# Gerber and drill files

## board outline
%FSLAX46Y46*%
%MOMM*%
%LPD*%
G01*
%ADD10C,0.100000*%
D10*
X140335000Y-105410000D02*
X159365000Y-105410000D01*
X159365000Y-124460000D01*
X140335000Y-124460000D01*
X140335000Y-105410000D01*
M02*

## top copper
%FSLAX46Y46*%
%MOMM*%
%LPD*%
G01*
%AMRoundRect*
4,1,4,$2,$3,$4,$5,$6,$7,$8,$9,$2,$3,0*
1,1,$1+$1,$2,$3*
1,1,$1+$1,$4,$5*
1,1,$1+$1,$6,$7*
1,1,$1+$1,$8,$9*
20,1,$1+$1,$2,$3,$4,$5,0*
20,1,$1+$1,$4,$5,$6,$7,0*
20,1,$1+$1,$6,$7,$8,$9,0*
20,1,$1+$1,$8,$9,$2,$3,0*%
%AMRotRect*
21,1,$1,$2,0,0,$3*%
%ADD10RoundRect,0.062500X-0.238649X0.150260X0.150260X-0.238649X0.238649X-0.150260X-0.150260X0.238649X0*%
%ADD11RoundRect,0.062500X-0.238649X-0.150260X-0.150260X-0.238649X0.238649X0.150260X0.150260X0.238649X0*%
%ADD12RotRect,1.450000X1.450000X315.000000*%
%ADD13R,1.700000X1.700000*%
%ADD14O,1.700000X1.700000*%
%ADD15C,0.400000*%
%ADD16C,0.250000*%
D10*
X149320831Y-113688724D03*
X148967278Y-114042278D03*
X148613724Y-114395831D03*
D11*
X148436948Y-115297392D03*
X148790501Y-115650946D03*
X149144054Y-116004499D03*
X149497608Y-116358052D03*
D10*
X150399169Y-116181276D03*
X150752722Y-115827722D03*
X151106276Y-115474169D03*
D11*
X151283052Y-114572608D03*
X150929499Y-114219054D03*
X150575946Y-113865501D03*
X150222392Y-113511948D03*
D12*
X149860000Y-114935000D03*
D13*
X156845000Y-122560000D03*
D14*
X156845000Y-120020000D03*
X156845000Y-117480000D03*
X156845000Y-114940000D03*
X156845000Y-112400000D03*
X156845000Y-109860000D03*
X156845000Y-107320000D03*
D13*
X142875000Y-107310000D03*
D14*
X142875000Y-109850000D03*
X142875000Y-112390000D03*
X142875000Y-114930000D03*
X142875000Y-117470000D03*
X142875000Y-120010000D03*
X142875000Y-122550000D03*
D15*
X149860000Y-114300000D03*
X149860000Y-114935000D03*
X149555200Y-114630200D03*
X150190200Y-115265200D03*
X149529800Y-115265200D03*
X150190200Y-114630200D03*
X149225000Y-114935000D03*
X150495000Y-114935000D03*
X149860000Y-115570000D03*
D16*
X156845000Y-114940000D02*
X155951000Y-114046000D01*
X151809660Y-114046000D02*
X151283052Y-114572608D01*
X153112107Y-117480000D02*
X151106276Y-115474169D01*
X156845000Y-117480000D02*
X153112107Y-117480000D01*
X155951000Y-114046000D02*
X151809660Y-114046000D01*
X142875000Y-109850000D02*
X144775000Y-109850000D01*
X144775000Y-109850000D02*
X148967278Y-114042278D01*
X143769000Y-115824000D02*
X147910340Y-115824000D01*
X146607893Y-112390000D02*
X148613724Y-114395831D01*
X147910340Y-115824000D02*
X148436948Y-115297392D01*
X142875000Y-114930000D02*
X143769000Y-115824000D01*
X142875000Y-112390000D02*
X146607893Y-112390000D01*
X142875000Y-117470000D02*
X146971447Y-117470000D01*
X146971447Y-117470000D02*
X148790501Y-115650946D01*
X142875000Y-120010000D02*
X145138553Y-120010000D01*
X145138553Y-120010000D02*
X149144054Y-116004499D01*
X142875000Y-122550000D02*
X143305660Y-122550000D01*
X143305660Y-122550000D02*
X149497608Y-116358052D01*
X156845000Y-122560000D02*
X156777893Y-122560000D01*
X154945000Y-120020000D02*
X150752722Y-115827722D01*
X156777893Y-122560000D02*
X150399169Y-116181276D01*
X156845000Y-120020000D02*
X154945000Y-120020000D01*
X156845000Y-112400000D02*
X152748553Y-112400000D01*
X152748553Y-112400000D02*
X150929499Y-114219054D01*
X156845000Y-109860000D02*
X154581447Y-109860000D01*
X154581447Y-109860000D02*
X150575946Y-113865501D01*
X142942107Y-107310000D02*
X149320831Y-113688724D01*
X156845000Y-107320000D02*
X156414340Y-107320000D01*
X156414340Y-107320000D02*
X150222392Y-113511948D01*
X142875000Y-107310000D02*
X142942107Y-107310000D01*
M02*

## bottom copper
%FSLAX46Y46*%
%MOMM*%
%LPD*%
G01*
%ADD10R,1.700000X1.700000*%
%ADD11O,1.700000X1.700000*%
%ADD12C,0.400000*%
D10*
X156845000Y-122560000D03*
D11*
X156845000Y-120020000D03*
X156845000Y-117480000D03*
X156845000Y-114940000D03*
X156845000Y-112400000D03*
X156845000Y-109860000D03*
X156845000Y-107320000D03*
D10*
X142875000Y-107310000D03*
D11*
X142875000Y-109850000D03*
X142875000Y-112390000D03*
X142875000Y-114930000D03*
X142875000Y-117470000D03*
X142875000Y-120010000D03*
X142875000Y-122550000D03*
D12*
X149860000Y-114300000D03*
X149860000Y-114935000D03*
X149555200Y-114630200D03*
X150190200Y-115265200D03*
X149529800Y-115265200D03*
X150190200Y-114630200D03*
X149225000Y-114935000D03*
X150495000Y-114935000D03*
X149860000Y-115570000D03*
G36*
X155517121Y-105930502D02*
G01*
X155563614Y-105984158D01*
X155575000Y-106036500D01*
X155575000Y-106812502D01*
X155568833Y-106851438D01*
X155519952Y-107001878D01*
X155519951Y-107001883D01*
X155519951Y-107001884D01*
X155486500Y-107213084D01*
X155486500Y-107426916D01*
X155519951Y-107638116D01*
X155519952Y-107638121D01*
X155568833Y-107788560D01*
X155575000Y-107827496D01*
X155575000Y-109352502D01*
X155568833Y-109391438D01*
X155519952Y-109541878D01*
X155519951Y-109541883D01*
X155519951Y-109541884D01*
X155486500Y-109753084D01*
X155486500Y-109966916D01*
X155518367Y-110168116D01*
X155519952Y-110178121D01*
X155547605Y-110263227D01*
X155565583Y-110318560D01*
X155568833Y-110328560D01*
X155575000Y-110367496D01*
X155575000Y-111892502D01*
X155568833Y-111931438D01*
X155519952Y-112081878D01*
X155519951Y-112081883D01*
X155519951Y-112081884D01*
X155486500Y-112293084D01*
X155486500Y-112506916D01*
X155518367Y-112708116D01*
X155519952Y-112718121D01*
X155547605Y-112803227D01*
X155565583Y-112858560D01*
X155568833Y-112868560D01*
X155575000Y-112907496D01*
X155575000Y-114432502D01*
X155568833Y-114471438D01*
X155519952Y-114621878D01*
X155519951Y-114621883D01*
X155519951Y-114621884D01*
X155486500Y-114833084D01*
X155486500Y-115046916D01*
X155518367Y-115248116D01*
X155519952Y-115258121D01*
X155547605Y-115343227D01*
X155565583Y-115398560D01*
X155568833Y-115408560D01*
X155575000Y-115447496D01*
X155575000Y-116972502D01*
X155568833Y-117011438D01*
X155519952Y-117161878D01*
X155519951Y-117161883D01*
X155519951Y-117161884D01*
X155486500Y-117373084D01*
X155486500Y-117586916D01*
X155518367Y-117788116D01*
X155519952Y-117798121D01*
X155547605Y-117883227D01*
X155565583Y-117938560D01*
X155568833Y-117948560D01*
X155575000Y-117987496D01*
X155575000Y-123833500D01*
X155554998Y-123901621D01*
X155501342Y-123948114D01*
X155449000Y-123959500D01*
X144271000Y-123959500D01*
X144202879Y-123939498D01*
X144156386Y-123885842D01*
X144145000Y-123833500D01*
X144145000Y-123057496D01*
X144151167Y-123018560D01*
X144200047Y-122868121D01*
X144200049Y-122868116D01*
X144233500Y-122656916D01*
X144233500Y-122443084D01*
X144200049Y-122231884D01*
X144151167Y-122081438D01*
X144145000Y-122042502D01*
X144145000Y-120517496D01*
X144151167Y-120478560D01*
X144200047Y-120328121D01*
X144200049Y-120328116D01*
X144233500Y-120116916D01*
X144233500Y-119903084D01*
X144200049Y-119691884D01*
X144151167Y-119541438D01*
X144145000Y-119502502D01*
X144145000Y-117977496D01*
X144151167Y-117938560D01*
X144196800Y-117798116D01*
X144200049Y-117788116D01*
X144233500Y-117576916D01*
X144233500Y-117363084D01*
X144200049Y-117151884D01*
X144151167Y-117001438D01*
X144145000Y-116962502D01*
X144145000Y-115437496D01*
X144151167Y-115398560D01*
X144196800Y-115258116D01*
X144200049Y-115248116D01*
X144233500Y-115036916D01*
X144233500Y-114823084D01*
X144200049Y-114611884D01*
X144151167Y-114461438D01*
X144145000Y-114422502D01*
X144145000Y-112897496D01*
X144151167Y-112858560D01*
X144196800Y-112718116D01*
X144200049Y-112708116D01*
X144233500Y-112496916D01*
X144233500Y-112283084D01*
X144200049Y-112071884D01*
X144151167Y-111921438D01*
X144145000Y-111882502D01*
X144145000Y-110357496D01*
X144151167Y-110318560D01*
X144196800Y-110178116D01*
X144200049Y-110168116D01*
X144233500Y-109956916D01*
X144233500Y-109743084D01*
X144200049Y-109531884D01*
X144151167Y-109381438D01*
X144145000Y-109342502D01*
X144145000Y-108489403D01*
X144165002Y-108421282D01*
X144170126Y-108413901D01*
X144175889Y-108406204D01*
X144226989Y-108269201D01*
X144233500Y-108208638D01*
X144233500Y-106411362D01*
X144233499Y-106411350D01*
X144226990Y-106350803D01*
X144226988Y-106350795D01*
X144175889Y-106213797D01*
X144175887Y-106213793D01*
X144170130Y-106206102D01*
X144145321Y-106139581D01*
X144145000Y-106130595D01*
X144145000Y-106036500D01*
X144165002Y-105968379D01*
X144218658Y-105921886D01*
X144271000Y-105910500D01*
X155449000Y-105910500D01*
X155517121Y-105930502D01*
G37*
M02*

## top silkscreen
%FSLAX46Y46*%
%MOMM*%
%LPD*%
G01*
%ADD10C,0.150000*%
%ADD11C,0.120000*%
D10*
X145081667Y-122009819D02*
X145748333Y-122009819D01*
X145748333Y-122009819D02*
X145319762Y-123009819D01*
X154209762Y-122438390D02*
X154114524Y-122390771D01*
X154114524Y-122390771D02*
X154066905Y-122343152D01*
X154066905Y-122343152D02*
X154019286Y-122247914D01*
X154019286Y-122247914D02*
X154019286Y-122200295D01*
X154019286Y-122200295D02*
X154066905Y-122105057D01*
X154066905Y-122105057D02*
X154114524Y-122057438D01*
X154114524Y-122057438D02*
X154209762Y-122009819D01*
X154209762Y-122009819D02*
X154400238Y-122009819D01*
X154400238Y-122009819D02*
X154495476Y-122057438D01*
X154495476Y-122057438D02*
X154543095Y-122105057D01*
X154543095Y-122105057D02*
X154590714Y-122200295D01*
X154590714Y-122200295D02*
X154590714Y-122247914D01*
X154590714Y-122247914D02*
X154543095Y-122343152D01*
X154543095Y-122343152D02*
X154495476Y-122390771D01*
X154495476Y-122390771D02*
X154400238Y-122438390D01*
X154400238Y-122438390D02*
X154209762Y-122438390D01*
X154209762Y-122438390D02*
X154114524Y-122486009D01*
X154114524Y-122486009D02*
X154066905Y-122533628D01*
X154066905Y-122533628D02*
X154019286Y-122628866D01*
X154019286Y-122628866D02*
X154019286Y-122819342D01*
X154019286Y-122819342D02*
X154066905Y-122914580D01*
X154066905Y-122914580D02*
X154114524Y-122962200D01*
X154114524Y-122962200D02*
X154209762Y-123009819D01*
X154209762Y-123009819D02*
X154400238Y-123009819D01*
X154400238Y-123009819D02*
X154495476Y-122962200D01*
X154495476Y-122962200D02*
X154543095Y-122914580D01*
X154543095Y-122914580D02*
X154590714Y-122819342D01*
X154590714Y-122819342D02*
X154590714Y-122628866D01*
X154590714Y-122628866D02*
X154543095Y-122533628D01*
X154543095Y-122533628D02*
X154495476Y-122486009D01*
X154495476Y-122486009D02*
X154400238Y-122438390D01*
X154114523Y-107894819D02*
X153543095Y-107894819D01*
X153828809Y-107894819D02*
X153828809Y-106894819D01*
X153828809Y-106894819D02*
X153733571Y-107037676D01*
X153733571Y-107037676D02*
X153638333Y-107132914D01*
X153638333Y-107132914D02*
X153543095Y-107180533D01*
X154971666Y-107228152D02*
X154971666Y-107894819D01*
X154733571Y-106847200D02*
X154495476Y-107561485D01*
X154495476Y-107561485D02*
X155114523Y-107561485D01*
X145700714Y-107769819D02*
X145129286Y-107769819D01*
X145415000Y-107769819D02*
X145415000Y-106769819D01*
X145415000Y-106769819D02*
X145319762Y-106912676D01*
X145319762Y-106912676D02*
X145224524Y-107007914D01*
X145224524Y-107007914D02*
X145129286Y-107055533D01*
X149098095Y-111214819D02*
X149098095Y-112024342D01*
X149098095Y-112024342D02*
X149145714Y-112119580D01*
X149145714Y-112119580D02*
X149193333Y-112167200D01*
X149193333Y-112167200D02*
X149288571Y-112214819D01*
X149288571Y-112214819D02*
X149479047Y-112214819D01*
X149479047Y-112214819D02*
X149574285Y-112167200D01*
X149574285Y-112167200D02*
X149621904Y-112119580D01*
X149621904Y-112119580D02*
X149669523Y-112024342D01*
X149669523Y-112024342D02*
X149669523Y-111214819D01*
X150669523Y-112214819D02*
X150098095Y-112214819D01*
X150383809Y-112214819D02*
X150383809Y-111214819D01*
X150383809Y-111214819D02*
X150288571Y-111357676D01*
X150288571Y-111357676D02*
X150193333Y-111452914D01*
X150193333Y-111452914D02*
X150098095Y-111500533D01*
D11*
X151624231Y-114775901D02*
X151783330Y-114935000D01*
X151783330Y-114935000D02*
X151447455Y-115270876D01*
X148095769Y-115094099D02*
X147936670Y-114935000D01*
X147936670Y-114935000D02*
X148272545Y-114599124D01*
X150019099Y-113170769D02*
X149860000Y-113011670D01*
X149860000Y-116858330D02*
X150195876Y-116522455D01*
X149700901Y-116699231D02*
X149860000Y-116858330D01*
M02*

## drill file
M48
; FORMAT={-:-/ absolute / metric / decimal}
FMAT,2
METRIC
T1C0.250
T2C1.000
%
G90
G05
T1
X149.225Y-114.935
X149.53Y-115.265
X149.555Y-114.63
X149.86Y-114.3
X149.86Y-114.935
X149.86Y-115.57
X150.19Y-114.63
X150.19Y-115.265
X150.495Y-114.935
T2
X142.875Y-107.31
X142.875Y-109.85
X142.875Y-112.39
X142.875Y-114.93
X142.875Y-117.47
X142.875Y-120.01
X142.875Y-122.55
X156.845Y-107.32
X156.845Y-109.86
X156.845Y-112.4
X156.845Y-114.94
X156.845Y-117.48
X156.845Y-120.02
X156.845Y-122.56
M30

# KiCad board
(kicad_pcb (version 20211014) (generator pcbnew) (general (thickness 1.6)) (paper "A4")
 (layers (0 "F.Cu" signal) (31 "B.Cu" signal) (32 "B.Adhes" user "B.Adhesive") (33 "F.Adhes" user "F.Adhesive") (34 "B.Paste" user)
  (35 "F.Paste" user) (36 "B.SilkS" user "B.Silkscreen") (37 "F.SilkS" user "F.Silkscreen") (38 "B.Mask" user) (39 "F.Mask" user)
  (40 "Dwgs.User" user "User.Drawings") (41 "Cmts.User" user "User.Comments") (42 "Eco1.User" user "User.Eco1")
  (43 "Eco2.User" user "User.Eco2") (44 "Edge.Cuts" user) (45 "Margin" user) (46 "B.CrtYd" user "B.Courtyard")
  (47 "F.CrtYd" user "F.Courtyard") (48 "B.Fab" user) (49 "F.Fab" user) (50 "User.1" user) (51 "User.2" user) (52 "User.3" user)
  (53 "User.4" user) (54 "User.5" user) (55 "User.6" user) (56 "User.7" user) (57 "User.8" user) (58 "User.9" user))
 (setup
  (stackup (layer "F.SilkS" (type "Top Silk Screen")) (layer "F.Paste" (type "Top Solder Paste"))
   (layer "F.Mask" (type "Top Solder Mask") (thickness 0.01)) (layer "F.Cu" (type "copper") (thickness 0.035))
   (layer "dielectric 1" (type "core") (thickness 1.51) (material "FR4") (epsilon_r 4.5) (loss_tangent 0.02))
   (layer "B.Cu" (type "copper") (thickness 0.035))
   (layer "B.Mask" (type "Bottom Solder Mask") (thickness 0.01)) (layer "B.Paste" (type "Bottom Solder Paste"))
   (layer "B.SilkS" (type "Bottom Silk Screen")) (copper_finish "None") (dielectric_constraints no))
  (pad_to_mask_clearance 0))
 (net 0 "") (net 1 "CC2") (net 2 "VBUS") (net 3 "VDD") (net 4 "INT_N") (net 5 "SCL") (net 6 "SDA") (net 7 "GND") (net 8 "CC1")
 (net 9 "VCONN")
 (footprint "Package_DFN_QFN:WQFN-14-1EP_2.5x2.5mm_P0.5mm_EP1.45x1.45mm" (layer "F.Cu") (at 149.86 114.935 -45)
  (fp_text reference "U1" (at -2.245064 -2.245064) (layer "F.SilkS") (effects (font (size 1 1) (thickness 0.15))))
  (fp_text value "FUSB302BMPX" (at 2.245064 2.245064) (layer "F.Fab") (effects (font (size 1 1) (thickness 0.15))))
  (fp_line (start 1.135 -1.36) (end 1.36 -1.36) (layer "F.SilkS") (width 0.12))
  (fp_line (start 1.36 -1.36) (end 1.36 -0.885) (layer "F.SilkS") (width 0.12))
  (fp_line (start -1.135 1.36) (end -1.36 1.36) (layer "F.SilkS") (width 0.12))
  (fp_line (start -1.36 1.36) (end -1.36 0.885) (layer "F.SilkS") (width 0.12))
  (fp_line (start -1.135 -1.36) (end -1.36 -1.36) (layer "F.SilkS") (width 0.12))
  (fp_line (start 1.36 1.36) (end 1.36 0.885) (layer "F.SilkS") (width 0.12))
  (fp_line (start 1.135 1.36) (end 1.36 1.36) (layer "F.SilkS") (width 0.12))
  (pad "" smd roundrect (at -0.36 0.36 315) (size 0.58 0.58) (layers "F.Paste") (roundrect_rratio 0.25))
  (pad "" smd roundrect (at 0.36 0.36 315) (size 0.58 0.58) (layers "F.Paste") (roundrect_rratio 0.25))
  (pad "" smd roundrect (at 0.36 -0.36 315) (size 0.58 0.58) (layers "F.Paste") (roundrect_rratio 0.25))
  (pad "" smd roundrect (at -0.36 -0.36 315) (size 0.58 0.58) (layers "F.Paste") (roundrect_rratio 0.25))
  (pad "1" smd roundrect (at -1.2625 -0.5 315) (size 0.675 0.25) (layers "F.Cu" "F.Paste" "F.Mask") (roundrect_rratio 0.25) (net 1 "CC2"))
  (pad "2" smd roundrect (at -1.2625 0 315) (size 0.675 0.25) (layers "F.Cu" "F.Paste" "F.Mask") (roundrect_rratio 0.25) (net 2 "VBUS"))
  (pad "3" smd roundrect (at -1.2625 0.5 315) (size 0.675 0.25) (layers "F.Cu" "F.Paste" "F.Mask") (roundrect_rratio 0.25) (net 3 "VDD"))
  (pad "4" smd roundrect (at -0.75 1.2625 315) (size 0.25 0.675) (layers "F.Cu" "F.Paste" "F.Mask") (roundrect_rratio 0.25) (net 3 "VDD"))
  (pad "5" smd roundrect (at -0.25 1.2625 315) (size 0.25 0.675) (layers "F.Cu" "F.Paste" "F.Mask") (roundrect_rratio 0.25) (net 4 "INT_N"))
  (pad "6" smd roundrect (at 0.25 1.2625 315) (size 0.25 0.675) (layers "F.Cu" "F.Paste" "F.Mask") (roundrect_rratio 0.25) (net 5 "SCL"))
  (pad "7" smd roundrect (at 0.75 1.2625 315) (size 0.25 0.675) (layers "F.Cu" "F.Paste" "F.Mask") (roundrect_rratio 0.25) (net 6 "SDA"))
  (pad "8" smd roundrect (at 1.2625 0.5 315) (size 0.675 0.25) (layers "F.Cu" "F.Paste" "F.Mask") (roundrect_rratio 0.25) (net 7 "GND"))
  (pad "9" smd roundrect (at 1.2625 0 315) (size 0.675 0.25) (layers "F.Cu" "F.Paste" "F.Mask") (roundrect_rratio 0.25) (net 7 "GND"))
  (pad "10" smd roundrect (at 1.2625 -0.5 315) (size 0.675 0.25) (layers "F.Cu" "F.Paste" "F.Mask") (roundrect_rratio 0.25) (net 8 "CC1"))
  (pad "11" smd roundrect (at 0.75 -1.2625 315) (size 0.25 0.675) (layers "F.Cu" "F.Paste" "F.Mask") (roundrect_rratio 0.25) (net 8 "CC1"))
  (pad "12" smd roundrect (at 0.25 -1.2625 315) (size 0.25 0.675) (layers "F.Cu" "F.Paste" "F.Mask") (roundrect_rratio 0.25) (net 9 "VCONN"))
  (pad "13" smd roundrect (at -0.25 -1.2625 315) (size 0.25 0.675) (layers "F.Cu" "F.Paste" "F.Mask") (roundrect_rratio 0.25)
   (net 9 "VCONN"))
  (pad "14" smd roundrect (at -0.75 -1.2625 315) (size 0.25 0.675) (layers "F.Cu" "F.Paste" "F.Mask") (roundrect_rratio 0.25) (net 1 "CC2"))
  (pad "15" smd rect (at 0 0 315) (size 1.45 1.45) (layers "F.Cu" "F.Mask") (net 7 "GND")))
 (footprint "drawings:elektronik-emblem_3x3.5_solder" (layer "B.Cu") (at 149.86 109.22 180)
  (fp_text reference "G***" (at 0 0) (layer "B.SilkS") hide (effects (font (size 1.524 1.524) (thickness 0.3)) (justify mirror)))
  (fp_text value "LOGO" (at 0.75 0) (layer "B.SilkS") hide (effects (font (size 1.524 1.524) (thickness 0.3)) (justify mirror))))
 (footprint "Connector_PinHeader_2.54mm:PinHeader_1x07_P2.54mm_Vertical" (layer "B.Cu") (at 156.845 122.56)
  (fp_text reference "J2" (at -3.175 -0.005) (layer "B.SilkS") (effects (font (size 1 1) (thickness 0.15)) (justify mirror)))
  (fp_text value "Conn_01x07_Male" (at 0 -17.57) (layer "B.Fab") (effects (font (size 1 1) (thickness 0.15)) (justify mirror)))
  (pad "1" thru_hole rect (at 0 0) (size 1.7 1.7) (drill 1) (layers *.Cu *.Mask) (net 7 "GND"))
  (pad "2" thru_hole oval (at 0 -2.54) (size 1.7 1.7) (drill 1) (layers *.Cu *.Mask) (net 7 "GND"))
  (pad "3" thru_hole oval (at 0 -5.08) (size 1.7 1.7) (drill 1) (layers *.Cu *.Mask) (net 8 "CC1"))
  (pad "4" thru_hole oval (at 0 -7.62) (size 1.7 1.7) (drill 1) (layers *.Cu *.Mask) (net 8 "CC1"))
  (pad "5" thru_hole oval (at 0 -10.16) (size 1.7 1.7) (drill 1) (layers *.Cu *.Mask) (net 9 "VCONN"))
  (pad "6" thru_hole oval (at 0 -12.7) (size 1.7 1.7) (drill 1) (layers *.Cu *.Mask) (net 9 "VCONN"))
  (pad "7" thru_hole oval (at 0 -15.24) (size 1.7 1.7) (drill 1) (layers *.Cu *.Mask) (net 1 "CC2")))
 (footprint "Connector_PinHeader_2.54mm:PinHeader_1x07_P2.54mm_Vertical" (layer "B.Cu") (at 142.875 107.31 180)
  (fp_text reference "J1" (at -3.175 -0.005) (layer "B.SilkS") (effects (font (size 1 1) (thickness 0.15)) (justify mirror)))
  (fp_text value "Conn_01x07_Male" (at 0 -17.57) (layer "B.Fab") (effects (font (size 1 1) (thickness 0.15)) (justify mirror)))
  (pad "1" thru_hole rect (at 0 0 180) (size 1.7 1.7) (drill 1) (layers *.Cu *.Mask) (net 1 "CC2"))
  (pad "2" thru_hole oval (at 0 -2.54 180) (size 1.7 1.7) (drill 1) (layers *.Cu *.Mask) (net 2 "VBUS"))
  (pad "3" thru_hole oval (at 0 -5.08 180) (size 1.7 1.7) (drill 1) (layers *.Cu *.Mask) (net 3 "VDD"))
  (pad "4" thru_hole oval (at 0 -7.62 180) (size 1.7 1.7) (drill 1) (layers *.Cu *.Mask) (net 3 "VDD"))
  (pad "5" thru_hole oval (at 0 -10.16 180) (size 1.7 1.7) (drill 1) (layers *.Cu *.Mask) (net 4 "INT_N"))
  (pad "6" thru_hole oval (at 0 -12.7 180) (size 1.7 1.7) (drill 1) (layers *.Cu *.Mask) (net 5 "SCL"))
  (pad "7" thru_hole oval (at 0 -15.24 180) (size 1.7 1.7) (drill 1) (layers *.Cu *.Mask) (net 6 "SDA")))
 (gr_rect (start 140.335 105.41) (end 159.365 124.46) (layer "Edge.Cuts") (width 0.1) (fill none))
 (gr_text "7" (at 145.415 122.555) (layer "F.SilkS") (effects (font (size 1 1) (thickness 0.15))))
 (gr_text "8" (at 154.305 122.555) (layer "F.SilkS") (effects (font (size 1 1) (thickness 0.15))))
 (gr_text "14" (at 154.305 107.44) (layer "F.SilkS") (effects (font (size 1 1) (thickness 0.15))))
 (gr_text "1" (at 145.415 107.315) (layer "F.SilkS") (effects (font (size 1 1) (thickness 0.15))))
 (segment (start 156.845 114.94) (end 155.951 114.046) (width 0.25) (layer "F.Cu") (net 8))
 (segment (start 151.80966 114.046) (end 151.283052 114.572608) (width 0.25) (layer "F.Cu") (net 8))
 (segment (start 153.112107 117.48) (end 151.106276 115.474169) (width 0.25) (layer "F.Cu") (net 8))
 (segment (start 156.845 117.48) (end 153.112107 117.48) (width 0.25) (layer "F.Cu") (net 8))
 (segment (start 155.951 114.046) (end 151.80966 114.046) (width 0.25) (layer "F.Cu") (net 8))
 (segment (start 142.875 109.85) (end 144.775 109.85) (width 0.25) (layer "F.Cu") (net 2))
 (segment (start 144.775 109.85) (end 148.967278 114.042278) (width 0.25) (layer "F.Cu") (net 2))
 (segment (start 143.769 115.824) (end 147.91034 115.824) (width 0.25) (layer "F.Cu") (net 3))
 (segment (start 146.607893 112.39) (end 148.613724 114.395831) (width 0.25) (layer "F.Cu") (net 3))
 (segment (start 147.91034 115.824) (end 148.436948 115.297392) (width 0.25) (layer "F.Cu") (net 3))
 (segment (start 142.875 114.93) (end 143.769 115.824) (width 0.25) (layer "F.Cu") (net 3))
 (segment (start 142.875 112.39) (end 146.607893 112.39) (width 0.25) (layer "F.Cu") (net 3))
 (segment (start 142.875 117.47) (end 146.971447 117.47) (width 0.25) (layer "F.Cu") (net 4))
 (segment (start 146.971447 117.47) (end 148.790501 115.650946) (width 0.25) (layer "F.Cu") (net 4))
 (segment (start 142.875 120.01) (end 145.138553 120.01) (width 0.25) (layer "F.Cu") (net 5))
 (segment (start 145.138553 120.01) (end 149.144054 116.004499) (width 0.25) (layer "F.Cu") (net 5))
 (segment (start 142.875 122.55) (end 143.30566 122.55) (width 0.25) (layer "F.Cu") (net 6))
 (segment (start 143.30566 122.55) (end 149.497608 116.358052) (width 0.25) (layer "F.Cu") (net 6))
 (segment (start 156.845 122.56) (end 156.777893 122.56) (width 0.25) (layer "F.Cu") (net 7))
 (segment (start 154.945 120.02) (end 150.752722 115.827722) (width 0.25) (layer "F.Cu") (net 7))
 (segment (start 156.777893 122.56) (end 150.399169 116.181276) (width 0.25) (layer "F.Cu") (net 7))
 (segment (start 156.845 120.02) (end 154.945 120.02) (width 0.25) (layer "F.Cu") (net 7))
 (via (at 149.86 114.3) (size 0.4) (drill 0.25) (layers "F.Cu" "B.Cu") (free) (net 7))
 (via (at 149.86 114.935) (size 0.4) (drill 0.25) (layers "F.Cu" "B.Cu") (free) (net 7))
 (via (at 149.5552 114.6302) (size 0.4) (drill 0.25) (layers "F.Cu" "B.Cu") (free) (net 7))
 (via (at 150.1902 115.2652) (size 0.4) (drill 0.25) (layers "F.Cu" "B.Cu") (free) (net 7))
 (via (at 149.5298 115.2652) (size 0.4) (drill 0.25) (layers "F.Cu" "B.Cu") (free) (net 7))
 (via (at 150.1902 114.6302) (size 0.4) (drill 0.25) (layers "F.Cu" "B.Cu") (free) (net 7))
 (via (at 149.225 114.935) (size 0.4) (drill 0.25) (layers "F.Cu" "B.Cu") (free) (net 7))
 (via (at 150.495 114.935) (size 0.4) (drill 0.25) (layers "F.Cu" "B.Cu") (free) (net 7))
 (via (at 149.86 115.57) (size 0.4) (drill 0.25) (layers "F.Cu" "B.Cu") (free) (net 7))
 (segment (start 156.845 112.4) (end 152.748553 112.4) (width 0.25) (layer "F.Cu") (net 9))
 (segment (start 152.748553 112.4) (end 150.929499 114.219054) (width 0.25) (layer "F.Cu") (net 9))
 (segment (start 156.845 109.86) (end 154.581447 109.86) (width 0.25) (layer "F.Cu") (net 9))
 (segment (start 154.581447 109.86) (end 150.575946 113.865501) (width 0.25) (layer "F.Cu") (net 9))
 (segment (start 142.942107 107.31) (end 149.320831 113.688724) (width 0.25) (layer "F.Cu") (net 1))
 (segment (start 156.845 107.32) (end 156.41434 107.32) (width 0.25) (layer "F.Cu") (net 1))
 (segment (start 156.41434 107.32) (end 150.222392 113.511948) (width 0.25) (layer "F.Cu") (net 1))
 (segment (start 142.875 107.31) (end 142.942107 107.31) (width 0.25) (layer "F.Cu") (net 1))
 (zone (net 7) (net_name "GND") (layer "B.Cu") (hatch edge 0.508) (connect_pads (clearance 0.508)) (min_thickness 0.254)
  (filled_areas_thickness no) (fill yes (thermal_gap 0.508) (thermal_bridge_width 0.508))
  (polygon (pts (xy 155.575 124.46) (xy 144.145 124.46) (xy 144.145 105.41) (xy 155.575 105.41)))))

